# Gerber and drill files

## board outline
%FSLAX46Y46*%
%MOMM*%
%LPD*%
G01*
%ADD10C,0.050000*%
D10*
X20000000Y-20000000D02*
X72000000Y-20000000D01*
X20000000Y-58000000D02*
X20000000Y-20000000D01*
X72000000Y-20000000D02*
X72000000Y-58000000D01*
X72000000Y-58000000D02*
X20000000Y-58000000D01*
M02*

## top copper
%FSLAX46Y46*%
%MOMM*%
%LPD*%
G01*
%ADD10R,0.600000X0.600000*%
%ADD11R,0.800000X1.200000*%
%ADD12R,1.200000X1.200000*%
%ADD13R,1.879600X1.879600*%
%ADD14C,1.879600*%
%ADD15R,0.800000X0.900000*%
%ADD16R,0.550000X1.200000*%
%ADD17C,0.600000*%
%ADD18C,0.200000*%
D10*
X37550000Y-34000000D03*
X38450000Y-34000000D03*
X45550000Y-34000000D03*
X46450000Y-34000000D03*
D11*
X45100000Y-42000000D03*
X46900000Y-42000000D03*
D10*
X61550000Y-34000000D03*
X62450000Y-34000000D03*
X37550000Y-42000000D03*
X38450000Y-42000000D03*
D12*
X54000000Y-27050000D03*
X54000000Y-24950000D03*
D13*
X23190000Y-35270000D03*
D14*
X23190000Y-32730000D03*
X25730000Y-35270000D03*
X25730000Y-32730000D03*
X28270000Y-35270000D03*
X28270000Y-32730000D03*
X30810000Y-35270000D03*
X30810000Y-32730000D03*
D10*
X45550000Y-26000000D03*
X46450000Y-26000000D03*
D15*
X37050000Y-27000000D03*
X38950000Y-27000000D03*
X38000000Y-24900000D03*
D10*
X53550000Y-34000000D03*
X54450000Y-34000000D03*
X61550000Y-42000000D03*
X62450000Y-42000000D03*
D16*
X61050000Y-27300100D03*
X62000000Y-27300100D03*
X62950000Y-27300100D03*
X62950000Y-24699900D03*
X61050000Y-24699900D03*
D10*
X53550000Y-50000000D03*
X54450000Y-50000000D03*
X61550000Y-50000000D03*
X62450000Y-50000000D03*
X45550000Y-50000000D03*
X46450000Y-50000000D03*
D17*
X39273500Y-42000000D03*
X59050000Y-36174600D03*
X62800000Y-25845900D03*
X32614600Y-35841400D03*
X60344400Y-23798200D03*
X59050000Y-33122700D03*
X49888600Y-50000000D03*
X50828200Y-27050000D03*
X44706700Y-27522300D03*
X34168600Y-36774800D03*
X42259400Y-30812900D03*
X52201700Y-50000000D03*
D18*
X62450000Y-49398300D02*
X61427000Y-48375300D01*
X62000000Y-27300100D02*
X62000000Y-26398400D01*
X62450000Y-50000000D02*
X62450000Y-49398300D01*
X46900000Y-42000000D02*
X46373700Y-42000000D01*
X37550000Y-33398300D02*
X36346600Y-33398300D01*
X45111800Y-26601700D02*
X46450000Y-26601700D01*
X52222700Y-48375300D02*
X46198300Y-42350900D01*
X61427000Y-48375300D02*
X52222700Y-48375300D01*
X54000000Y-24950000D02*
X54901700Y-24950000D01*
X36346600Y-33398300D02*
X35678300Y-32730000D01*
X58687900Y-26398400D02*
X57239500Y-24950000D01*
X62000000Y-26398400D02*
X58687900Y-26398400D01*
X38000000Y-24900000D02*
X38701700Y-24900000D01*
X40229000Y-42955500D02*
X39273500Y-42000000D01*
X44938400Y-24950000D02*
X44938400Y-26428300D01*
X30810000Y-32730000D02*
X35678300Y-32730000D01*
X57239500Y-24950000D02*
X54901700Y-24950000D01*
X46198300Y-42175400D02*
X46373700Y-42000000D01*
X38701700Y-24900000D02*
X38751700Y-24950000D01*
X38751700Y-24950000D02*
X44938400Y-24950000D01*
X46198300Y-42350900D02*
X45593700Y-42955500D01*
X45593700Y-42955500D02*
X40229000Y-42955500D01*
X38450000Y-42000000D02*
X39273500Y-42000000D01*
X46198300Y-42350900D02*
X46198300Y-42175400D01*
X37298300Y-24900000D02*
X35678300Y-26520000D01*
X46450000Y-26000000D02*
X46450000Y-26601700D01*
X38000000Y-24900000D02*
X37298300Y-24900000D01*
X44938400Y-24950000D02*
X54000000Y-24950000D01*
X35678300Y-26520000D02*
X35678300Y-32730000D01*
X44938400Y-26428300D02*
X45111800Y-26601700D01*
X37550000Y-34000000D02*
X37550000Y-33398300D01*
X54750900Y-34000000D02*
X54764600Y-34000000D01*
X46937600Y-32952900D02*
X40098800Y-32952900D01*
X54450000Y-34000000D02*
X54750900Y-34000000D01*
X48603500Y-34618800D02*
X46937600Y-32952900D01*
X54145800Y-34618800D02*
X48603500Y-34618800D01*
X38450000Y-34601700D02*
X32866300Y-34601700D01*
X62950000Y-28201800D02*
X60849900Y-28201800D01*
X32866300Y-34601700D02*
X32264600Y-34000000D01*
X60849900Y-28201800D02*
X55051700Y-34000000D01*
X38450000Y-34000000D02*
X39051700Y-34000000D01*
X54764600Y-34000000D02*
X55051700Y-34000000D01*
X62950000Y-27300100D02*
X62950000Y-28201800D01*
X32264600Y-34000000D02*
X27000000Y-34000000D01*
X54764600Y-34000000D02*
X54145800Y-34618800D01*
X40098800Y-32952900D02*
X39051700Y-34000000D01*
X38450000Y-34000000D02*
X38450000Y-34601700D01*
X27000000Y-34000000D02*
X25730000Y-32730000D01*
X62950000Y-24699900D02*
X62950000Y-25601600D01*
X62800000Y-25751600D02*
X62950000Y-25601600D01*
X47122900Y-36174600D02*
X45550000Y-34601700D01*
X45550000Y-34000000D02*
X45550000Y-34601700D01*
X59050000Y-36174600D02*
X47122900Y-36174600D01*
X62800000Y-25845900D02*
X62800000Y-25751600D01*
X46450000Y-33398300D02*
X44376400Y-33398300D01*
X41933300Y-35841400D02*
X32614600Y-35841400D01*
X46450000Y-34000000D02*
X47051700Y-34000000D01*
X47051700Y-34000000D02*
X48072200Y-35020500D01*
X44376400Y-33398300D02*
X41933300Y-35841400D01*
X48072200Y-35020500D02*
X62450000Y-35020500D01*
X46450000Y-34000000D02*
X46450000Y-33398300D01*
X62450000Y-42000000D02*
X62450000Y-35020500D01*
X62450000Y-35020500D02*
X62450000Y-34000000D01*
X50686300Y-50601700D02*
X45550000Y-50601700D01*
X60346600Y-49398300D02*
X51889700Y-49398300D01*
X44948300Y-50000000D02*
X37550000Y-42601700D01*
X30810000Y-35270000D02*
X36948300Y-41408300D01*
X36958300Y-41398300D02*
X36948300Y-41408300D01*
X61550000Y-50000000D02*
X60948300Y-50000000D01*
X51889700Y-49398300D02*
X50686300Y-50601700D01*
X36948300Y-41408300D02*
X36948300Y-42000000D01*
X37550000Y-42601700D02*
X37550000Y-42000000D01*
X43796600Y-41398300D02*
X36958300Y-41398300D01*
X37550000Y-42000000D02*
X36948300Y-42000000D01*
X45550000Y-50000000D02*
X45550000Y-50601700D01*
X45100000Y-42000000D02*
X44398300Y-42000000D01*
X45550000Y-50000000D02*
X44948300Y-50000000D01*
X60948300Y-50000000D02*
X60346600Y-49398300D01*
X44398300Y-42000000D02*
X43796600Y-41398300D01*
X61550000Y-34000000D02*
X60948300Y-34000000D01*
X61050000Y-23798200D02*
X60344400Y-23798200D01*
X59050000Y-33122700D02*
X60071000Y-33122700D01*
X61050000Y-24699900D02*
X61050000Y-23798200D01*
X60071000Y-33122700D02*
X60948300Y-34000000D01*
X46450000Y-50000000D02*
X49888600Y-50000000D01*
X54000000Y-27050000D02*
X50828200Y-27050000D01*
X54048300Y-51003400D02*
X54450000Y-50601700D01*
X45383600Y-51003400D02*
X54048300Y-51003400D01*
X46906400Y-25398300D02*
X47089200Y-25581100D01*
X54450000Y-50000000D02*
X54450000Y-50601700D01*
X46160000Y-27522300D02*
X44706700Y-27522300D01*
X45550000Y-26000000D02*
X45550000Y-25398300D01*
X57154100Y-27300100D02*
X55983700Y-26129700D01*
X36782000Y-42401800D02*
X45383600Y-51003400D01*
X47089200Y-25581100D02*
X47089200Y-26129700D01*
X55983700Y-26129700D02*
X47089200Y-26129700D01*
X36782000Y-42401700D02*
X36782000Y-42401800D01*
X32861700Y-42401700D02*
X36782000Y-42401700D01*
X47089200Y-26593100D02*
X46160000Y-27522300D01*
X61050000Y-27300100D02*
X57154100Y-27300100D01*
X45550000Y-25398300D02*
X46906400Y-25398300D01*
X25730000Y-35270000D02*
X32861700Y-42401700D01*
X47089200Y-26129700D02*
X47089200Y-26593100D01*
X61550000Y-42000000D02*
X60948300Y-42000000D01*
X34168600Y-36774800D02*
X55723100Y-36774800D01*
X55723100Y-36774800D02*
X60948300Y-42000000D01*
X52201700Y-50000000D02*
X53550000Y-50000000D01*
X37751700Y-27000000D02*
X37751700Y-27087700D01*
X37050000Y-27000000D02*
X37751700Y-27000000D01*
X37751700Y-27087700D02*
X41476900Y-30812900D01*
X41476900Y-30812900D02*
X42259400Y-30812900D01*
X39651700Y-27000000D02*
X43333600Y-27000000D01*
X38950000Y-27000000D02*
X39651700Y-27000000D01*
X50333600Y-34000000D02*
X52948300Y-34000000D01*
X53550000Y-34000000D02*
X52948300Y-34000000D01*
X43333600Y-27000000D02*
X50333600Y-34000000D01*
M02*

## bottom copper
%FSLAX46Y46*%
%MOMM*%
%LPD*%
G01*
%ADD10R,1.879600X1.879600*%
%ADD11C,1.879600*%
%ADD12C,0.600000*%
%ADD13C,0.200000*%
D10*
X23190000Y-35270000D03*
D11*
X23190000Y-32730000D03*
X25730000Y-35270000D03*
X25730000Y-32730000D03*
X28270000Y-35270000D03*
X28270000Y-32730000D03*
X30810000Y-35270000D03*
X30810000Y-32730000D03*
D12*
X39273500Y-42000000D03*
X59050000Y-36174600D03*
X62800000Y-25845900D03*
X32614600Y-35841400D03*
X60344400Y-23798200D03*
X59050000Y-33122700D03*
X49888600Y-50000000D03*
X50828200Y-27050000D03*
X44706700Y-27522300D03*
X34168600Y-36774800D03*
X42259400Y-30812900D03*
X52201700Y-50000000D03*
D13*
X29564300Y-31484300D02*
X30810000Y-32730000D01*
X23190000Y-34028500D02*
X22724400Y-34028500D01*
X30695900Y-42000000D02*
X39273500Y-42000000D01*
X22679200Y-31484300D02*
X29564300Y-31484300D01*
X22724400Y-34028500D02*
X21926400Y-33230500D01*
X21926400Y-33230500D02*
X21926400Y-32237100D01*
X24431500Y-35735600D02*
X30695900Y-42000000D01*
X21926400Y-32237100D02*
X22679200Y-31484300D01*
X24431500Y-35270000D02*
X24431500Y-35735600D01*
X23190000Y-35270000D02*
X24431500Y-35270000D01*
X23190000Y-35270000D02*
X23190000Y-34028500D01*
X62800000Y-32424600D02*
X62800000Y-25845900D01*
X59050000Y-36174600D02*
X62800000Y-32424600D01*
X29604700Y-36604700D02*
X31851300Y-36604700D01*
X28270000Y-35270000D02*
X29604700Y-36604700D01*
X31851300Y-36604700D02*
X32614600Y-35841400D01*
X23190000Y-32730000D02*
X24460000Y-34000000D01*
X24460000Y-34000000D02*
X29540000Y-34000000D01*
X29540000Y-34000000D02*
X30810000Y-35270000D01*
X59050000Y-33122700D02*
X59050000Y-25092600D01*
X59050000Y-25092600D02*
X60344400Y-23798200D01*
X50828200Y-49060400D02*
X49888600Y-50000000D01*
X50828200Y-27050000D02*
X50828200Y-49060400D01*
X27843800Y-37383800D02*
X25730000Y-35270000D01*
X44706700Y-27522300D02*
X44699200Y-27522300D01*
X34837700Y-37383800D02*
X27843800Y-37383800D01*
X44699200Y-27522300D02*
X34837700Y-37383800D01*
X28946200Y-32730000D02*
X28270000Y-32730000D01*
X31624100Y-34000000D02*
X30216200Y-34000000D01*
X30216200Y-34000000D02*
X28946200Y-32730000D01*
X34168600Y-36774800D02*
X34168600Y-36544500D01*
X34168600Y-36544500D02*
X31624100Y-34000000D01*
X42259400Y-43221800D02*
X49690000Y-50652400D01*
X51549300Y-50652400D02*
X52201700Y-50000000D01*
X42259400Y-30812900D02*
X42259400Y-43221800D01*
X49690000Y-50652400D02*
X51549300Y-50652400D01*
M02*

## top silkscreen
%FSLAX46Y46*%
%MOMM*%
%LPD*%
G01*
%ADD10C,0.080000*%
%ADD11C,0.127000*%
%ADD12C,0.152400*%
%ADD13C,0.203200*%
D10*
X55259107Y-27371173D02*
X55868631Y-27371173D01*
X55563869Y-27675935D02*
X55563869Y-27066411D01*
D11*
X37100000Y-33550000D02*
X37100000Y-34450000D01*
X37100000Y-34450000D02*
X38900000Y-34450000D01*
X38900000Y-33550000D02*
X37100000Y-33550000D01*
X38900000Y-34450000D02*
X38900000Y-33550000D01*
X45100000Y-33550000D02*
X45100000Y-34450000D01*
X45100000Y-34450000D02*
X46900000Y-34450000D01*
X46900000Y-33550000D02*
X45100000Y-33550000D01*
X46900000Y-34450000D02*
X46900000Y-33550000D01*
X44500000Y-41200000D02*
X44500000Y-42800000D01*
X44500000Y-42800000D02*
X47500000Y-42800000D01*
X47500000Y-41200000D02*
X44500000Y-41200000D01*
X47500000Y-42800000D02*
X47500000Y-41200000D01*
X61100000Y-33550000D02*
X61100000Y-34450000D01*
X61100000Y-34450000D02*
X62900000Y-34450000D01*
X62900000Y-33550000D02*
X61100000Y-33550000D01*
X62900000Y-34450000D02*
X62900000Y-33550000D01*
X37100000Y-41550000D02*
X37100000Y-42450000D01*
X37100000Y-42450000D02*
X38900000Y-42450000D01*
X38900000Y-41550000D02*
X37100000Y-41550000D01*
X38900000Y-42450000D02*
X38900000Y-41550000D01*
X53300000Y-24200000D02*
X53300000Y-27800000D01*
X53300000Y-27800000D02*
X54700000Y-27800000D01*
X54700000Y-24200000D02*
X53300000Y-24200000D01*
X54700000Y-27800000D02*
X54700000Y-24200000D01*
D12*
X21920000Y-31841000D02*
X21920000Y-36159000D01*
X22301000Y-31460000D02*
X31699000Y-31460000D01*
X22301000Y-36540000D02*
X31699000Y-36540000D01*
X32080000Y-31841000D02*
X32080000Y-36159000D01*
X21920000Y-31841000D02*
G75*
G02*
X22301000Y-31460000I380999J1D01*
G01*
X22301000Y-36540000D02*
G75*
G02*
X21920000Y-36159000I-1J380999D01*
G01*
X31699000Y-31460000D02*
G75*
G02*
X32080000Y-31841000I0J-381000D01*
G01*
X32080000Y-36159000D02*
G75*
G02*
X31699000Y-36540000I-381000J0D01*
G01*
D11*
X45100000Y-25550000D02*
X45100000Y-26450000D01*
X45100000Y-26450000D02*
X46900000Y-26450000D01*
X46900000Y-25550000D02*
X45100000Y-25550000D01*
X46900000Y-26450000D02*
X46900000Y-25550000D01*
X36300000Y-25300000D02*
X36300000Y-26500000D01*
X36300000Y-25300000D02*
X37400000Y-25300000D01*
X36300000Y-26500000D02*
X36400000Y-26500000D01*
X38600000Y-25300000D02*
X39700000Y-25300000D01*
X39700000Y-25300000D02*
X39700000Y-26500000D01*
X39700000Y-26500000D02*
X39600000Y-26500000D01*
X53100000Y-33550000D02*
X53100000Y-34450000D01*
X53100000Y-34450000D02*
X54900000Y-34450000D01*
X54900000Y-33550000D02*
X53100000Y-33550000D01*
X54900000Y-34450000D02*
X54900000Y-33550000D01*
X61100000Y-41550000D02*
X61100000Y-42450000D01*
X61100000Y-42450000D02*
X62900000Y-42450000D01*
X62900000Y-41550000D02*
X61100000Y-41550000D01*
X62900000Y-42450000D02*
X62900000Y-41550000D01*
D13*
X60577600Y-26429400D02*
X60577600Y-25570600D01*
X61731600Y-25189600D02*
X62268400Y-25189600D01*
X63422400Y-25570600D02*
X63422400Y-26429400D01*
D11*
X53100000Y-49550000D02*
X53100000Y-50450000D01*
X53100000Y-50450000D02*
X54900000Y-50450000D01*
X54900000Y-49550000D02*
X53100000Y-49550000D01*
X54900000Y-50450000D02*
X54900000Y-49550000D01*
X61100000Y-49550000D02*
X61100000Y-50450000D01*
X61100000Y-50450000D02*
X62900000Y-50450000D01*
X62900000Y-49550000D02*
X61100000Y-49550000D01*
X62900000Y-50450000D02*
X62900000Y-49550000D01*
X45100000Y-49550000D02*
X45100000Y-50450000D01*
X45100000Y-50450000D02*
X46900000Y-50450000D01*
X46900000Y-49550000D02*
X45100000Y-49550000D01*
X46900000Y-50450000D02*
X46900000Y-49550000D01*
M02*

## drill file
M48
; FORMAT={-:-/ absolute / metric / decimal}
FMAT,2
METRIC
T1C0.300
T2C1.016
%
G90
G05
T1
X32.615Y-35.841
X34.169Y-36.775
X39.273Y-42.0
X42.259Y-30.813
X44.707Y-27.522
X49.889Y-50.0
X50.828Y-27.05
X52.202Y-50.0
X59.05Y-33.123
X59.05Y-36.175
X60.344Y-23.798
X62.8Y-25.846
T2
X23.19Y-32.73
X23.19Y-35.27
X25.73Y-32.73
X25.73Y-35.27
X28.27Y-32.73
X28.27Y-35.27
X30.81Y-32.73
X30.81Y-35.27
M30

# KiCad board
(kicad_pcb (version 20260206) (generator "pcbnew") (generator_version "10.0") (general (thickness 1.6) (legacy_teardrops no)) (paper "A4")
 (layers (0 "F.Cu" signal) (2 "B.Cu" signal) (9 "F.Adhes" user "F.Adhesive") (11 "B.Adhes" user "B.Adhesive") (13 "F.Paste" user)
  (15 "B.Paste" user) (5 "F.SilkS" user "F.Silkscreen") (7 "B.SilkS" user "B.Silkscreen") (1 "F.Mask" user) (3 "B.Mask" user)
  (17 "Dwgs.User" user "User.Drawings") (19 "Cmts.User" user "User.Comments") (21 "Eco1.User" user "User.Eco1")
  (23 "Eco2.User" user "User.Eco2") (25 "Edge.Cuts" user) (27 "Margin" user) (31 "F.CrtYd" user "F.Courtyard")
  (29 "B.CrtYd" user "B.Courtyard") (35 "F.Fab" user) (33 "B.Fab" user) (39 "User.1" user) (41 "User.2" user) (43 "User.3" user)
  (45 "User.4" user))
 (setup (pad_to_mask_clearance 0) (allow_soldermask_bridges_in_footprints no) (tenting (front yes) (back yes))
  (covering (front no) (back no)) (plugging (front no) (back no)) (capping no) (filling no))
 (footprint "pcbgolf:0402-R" (layer "F.Cu") (at 38 34)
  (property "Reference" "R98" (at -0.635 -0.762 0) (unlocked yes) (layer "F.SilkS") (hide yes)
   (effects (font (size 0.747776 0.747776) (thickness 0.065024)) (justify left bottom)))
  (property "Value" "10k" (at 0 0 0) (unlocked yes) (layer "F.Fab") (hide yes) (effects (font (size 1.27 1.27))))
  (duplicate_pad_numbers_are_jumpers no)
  (fp_line (start -0.9 -0.45) (end -0.9 0.45) (stroke (width 0.127) (type solid)) (layer "F.SilkS"))
  (fp_line (start -0.9 0.45) (end 0.9 0.45) (stroke (width 0.127) (type solid)) (layer "F.SilkS"))
  (fp_line (start 0.9 -0.45) (end -0.9 -0.45) (stroke (width 0.127) (type solid)) (layer "F.SilkS"))
  (fp_line (start 0.9 0.45) (end 0.9 -0.45) (stroke (width 0.127) (type solid)) (layer "F.SilkS"))
  (pad "1" smd rect (at -0.45 0) (size 0.6 0.6) (layers "F.Cu" "F.Mask" "F.Paste") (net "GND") (solder_mask_margin 0.0508)
   (solder_paste_margin 0) (thermal_bridge_angle 0))
  (pad "2" smd rect (at 0.45 0) (size 0.6 0.6) (layers "F.Cu" "F.Mask" "F.Paste") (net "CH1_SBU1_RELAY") (solder_mask_margin 0.0508)
   (solder_paste_margin 0) (thermal_bridge_angle 0)))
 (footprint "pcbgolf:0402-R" (layer "F.Cu") (at 46 34)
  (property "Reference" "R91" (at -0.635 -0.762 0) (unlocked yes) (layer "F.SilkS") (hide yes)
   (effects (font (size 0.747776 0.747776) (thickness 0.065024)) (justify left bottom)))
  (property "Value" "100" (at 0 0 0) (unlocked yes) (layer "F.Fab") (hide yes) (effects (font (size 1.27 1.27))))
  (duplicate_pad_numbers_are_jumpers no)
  (fp_line (start -0.9 -0.45) (end -0.9 0.45) (stroke (width 0.127) (type solid)) (layer "F.SilkS"))
  (fp_line (start -0.9 0.45) (end 0.9 0.45) (stroke (width 0.127) (type solid)) (layer "F.SilkS"))
  (fp_line (start 0.9 -0.45) (end -0.9 -0.45) (stroke (width 0.127) (type solid)) (layer "F.SilkS"))
  (fp_line (start 0.9 0.45) (end 0.9 -0.45) (stroke (width 0.127) (type solid)) (layer "F.SilkS"))
  (pad "1" smd rect (at -0.45 0) (size 0.6 0.6) (layers "F.Cu" "F.Mask" "F.Paste") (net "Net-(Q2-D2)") (solder_mask_margin 0.0508)
   (solder_paste_margin 0) (thermal_bridge_angle 0))
  (pad "2" smd rect (at 0.45 0) (size 0.6 0.6) (layers "F.Cu" "F.Mask" "F.Paste") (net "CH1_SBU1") (solder_mask_margin 0.0508)
   (solder_paste_margin 0) (thermal_bridge_angle 0)))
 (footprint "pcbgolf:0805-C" (layer "F.Cu") (at 46 42)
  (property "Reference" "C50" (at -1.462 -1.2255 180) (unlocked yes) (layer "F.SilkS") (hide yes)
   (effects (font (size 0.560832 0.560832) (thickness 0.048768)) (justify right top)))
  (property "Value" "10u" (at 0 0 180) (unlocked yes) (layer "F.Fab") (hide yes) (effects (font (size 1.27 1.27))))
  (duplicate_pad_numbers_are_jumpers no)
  (fp_line (start -1.5 -0.8) (end -1.5 0.8) (stroke (width 0.127) (type solid)) (layer "F.SilkS"))
  (fp_line (start -1.5 0.8) (end 1.5 0.8) (stroke (width 0.127) (type solid)) (layer "F.SilkS"))
  (fp_line (start 1.5 -0.8) (end -1.5 -0.8) (stroke (width 0.127) (type solid)) (layer "F.SilkS"))
  (fp_line (start 1.5 0.8) (end 1.5 -0.8) (stroke (width 0.127) (type solid)) (layer "F.SilkS"))
  (pad "1" smd rect (at -0.9 0) (size 0.8 1.2) (layers "F.Cu" "F.Mask" "F.Paste") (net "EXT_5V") (solder_mask_margin 0.0508)
   (solder_paste_margin 0) (thermal_bridge_angle 0))
  (pad "2" smd rect (at 0.9 0) (size 0.8 1.2) (layers "F.Cu" "F.Mask" "F.Paste") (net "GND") (solder_mask_margin 0.0508)
   (solder_paste_margin 0) (thermal_bridge_angle 0)))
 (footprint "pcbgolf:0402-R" (layer "F.Cu") (at 62 34)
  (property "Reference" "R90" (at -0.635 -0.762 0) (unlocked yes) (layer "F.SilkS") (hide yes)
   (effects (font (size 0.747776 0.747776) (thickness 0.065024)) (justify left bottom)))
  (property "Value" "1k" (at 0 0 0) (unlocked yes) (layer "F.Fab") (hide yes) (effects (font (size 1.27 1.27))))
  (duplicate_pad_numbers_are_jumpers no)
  (fp_line (start -0.9 -0.45) (end -0.9 0.45) (stroke (width 0.127) (type solid)) (layer "F.SilkS"))
  (fp_line (start -0.9 0.45) (end 0.9 0.45) (stroke (width 0.127) (type solid)) (layer "F.SilkS"))
  (fp_line (start 0.9 -0.45) (end -0.9 -0.45) (stroke (width 0.127) (type solid)) (layer "F.SilkS"))
  (fp_line (start 0.9 0.45) (end 0.9 -0.45) (stroke (width 0.127) (type solid)) (layer "F.SilkS"))
  (pad "1" smd rect (at -0.45 0) (size 0.6 0.6) (layers "F.Cu" "F.Mask" "F.Paste") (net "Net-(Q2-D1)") (solder_mask_margin 0.0508)
   (solder_paste_margin 0) (thermal_bridge_angle 0))
  (pad "2" smd rect (at 0.45 0) (size 0.6 0.6) (layers "F.Cu" "F.Mask" "F.Paste") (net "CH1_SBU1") (solder_mask_margin 0.0508)
   (solder_paste_margin 0) (thermal_bridge_angle 0)))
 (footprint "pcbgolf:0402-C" (layer "F.Cu") (at 38 42)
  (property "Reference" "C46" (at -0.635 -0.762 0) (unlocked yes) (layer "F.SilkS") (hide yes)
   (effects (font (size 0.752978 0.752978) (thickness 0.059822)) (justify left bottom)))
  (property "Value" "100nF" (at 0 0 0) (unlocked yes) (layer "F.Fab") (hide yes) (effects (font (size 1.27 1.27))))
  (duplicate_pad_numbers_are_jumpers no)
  (fp_line (start -0.9 -0.45) (end -0.9 0.45) (stroke (width 0.127) (type solid)) (layer "F.SilkS"))
  (fp_line (start -0.9 0.45) (end 0.9 0.45) (stroke (width 0.127) (type solid)) (layer "F.SilkS"))
  (fp_line (start 0.9 -0.45) (end -0.9 -0.45) (stroke (width 0.127) (type solid)) (layer "F.SilkS"))
  (fp_line (start 0.9 0.45) (end 0.9 -0.45) (stroke (width 0.127) (type solid)) (layer "F.SilkS"))
  (pad "1" smd rect (at -0.45 0) (size 0.6 0.6) (layers "F.Cu" "F.Mask" "F.Paste") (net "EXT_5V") (solder_mask_margin 0.0508)
   (solder_paste_margin 0) (thermal_bridge_angle 0))
  (pad "2" smd rect (at 0.45 0) (size 0.6 0.6) (layers "F.Cu" "F.Mask" "F.Paste") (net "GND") (solder_mask_margin 0.0508)
   (solder_paste_margin 0) (thermal_bridge_angle 0)))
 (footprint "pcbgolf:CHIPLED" (layer "F.Cu") (at 54 26)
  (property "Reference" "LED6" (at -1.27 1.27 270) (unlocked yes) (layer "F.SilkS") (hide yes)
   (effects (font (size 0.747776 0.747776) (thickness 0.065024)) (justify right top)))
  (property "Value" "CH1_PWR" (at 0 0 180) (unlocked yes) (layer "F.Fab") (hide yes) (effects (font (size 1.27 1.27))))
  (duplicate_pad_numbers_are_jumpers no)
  (fp_line (start -0.7 -1.8) (end -0.7 1.8) (stroke (width 0.127) (type solid)) (layer "F.SilkS"))
  (fp_line (start -0.7 1.8) (end 0.7 1.8) (stroke (width 0.127) (type solid)) (layer "F.SilkS"))
  (fp_line (start 0.7 -1.8) (end -0.7 -1.8) (stroke (width 0.127) (type solid)) (layer "F.SilkS"))
  (fp_line (start 0.7 1.8) (end 0.7 -1.8) (stroke (width 0.127) (type solid)) (layer "F.SilkS"))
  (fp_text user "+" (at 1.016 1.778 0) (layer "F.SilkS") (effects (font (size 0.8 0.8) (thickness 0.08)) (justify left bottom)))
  (pad "A" smd rect (at 0 1.05) (size 1.2 1.2) (layers "F.Cu" "F.Mask" "F.Paste") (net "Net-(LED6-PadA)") (solder_mask_margin 0.0508)
   (solder_paste_margin 0) (thermal_bridge_angle 0))
  (pad "C" smd rect (at 0 -1.05) (size 1.2 1.2) (layers "F.Cu" "F.Mask" "F.Paste") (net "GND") (solder_mask_margin 0.0508)
   (solder_paste_margin 0) (thermal_bridge_angle 0)))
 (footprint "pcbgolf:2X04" (layer "F.Cu") (at 27 34)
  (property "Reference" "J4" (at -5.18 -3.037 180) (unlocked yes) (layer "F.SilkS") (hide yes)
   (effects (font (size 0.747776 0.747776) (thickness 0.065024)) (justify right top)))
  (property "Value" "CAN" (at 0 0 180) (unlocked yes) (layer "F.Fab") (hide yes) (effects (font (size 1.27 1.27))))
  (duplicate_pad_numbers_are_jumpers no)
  (fp_line (start -5.08 -2.159) (end -5.08 2.159) (stroke (width 0.1524) (type solid)) (layer "F.SilkS"))
  (fp_line (start -4.699 -2.54) (end 4.699 -2.54) (stroke (width 0.1524) (type solid)) (layer "F.SilkS"))
  (fp_line (start -4.699 2.54) (end 4.699 2.54) (stroke (width 0.1524) (type solid)) (layer "F.SilkS"))
  (fp_line (start 5.08 -2.159) (end 5.08 2.159) (stroke (width 0.1524) (type solid)) (layer "F.SilkS"))
  (fp_arc (start -5.08 -2.159) (mid -4.968408 -2.428408) (end -4.699 -2.54) (stroke (width 0.1524) (type solid)) (layer "F.SilkS"))
  (fp_arc (start -4.699 2.54) (mid -4.968408 2.428408) (end -5.08 2.159) (stroke (width 0.1524) (type solid)) (layer "F.SilkS"))
  (fp_arc (start 4.699 -2.54) (mid 4.968408 -2.428408) (end 5.08 -2.159) (stroke (width 0.1524) (type solid)) (layer "F.SilkS"))
  (fp_arc (start 5.08 2.159) (mid 4.968408 2.428408) (end 4.699 2.54) (stroke (width 0.1524) (type solid)) (layer "F.SilkS"))
  (pad "1" thru_hole rect (at -3.81 1.27 90) (size 1.8796 1.8796) (drill 1.016) (layers "*.Cu" "*.Mask") (remove_unused_layers no)
   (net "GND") (solder_mask_margin 0.0508) (thermal_bridge_angle 0))
  (pad "2" thru_hole circle (at -3.81 -1.27 90) (size 1.8796 1.8796) (drill 1.016) (layers "*.Cu" "*.Mask") (remove_unused_layers no)
   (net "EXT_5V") (solder_mask_margin 0.0508) (thermal_bridge_angle 0))
  (pad "3" thru_hole circle (at -1.27 1.27 90) (size 1.8796 1.8796) (drill 1.016) (layers "*.Cu" "*.Mask") (remove_unused_layers no)
   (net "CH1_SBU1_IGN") (solder_mask_margin 0.0508) (thermal_bridge_angle 0))
  (pad "4" thru_hole circle (at -1.27 -1.27 90) (size 1.8796 1.8796) (drill 1.016) (layers "*.Cu" "*.Mask") (remove_unused_layers no)
   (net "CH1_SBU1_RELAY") (solder_mask_margin 0.0508) (thermal_bridge_angle 0))
  (pad "5" thru_hole circle (at 1.27 1.27 90) (size 1.8796 1.8796) (drill 1.016) (layers "*.Cu" "*.Mask") (remove_unused_layers no)
   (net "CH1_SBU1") (solder_mask_margin 0.0508) (thermal_bridge_angle 0))
  (pad "6" thru_hole circle (at 1.27 -1.27 90) (size 1.8796 1.8796) (drill 1.016) (layers "*.Cu" "*.Mask") (remove_unused_layers no)
   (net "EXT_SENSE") (solder_mask_margin 0.0508) (thermal_bridge_angle 0))
  (pad "7" thru_hole circle (at 3.81 1.27 90) (size 1.8796 1.8796) (drill 1.016) (layers "*.Cu" "*.Mask") (remove_unused_layers no)
   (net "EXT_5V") (solder_mask_margin 0.0508) (thermal_bridge_angle 0))
  (pad "8" thru_hole circle (at 3.81 -1.27 90) (size 1.8796 1.8796) (drill 1.016) (layers "*.Cu" "*.Mask") (remove_unused_layers no)
   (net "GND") (solder_mask_margin 0.0508) (thermal_bridge_angle 0)))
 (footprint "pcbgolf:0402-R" (layer "F.Cu") (at 46 26)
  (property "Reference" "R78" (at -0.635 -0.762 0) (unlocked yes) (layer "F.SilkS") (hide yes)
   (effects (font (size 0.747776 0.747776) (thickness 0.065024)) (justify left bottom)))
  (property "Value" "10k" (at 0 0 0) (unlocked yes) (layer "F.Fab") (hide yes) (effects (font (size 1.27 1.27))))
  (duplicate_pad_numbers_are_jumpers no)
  (fp_line (start -0.9 -0.45) (end -0.9 0.45) (stroke (width 0.127) (type solid)) (layer "F.SilkS"))
  (fp_line (start -0.9 0.45) (end 0.9 0.45) (stroke (width 0.127) (type solid)) (layer "F.SilkS"))
  (fp_line (start 0.9 -0.45) (end -0.9 -0.45) (stroke (width 0.127) (type solid)) (layer "F.SilkS"))
  (fp_line (start 0.9 0.45) (end 0.9 -0.45) (stroke (width 0.127) (type solid)) (layer "F.SilkS"))
  (pad "1" smd rect (at -0.45 0) (size 0.6 0.6) (layers "F.Cu" "F.Mask" "F.Paste") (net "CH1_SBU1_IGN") (solder_mask_margin 0.0508)
   (solder_paste_margin 0) (thermal_bridge_angle 0))
  (pad "2" smd rect (at 0.45 0) (size 0.6 0.6) (layers "F.Cu" "F.Mask" "F.Paste") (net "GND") (solder_mask_margin 0.0508)
   (solder_paste_margin 0) (thermal_bridge_angle 0)))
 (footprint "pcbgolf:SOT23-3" (layer "F.Cu") (at 38 26)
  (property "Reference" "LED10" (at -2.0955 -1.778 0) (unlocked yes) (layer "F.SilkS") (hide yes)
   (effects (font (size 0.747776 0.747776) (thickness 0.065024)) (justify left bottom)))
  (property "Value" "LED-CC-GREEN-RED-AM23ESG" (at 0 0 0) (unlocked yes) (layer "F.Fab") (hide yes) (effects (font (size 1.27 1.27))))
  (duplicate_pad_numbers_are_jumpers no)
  (fp_line (start -1.7 -0.7) (end -1.7 0.5) (stroke (width 0.127) (type solid)) (layer "F.SilkS"))
  (fp_line (start -1.7 -0.7) (end -0.6 -0.7) (stroke (width 0.127) (type solid)) (layer "F.SilkS"))
  (fp_line (start -1.7 0.5) (end -1.6 0.5) (stroke (width 0.127) (type solid)) (layer "F.SilkS"))
  (fp_line (start 0.6 -0.7) (end 1.7 -0.7) (stroke (width 0.127) (type solid)) (layer "F.SilkS"))
  (fp_line (start 1.7 -0.7) (end 1.7 0.5) (stroke (width 0.127) (type solid)) (layer "F.SilkS"))
  (fp_line (start 1.7 0.5) (end 1.6 0.5) (stroke (width 0.127) (type solid)) (layer "F.SilkS"))
  (pad "1" smd rect (at -0.95 1) (size 0.8 0.9) (layers "F.Cu" "F.Mask" "F.Paste") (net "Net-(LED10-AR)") (solder_mask_margin 0.0508)
   (solder_paste_margin 0) (thermal_bridge_angle 0))
  (pad "2" smd rect (at 0.95 1) (size 0.8 0.9) (layers "F.Cu" "F.Mask" "F.Paste") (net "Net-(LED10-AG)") (solder_mask_margin 0.0508)
   (solder_paste_margin 0) (thermal_bridge_angle 0))
  (pad "3" smd rect (at 0 -1.1) (size 0.8 0.9) (layers "F.Cu" "F.Mask" "F.Paste") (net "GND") (solder_mask_margin 0.0508)
   (solder_paste_margin 0) (thermal_bridge_angle 0)))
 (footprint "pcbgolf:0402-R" (layer "F.Cu") (at 54 34)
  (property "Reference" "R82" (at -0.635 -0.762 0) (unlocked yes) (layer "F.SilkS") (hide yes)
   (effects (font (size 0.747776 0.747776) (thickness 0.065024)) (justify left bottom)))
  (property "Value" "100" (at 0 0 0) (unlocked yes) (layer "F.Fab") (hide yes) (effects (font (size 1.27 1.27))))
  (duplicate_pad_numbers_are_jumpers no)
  (fp_line (start -0.9 -0.45) (end -0.9 0.45) (stroke (width 0.127) (type solid)) (layer "F.SilkS"))
  (fp_line (start -0.9 0.45) (end 0.9 0.45) (stroke (width 0.127) (type solid)) (layer "F.SilkS"))
  (fp_line (start 0.9 -0.45) (end -0.9 -0.45) (stroke (width 0.127) (type solid)) (layer "F.SilkS"))
  (fp_line (start 0.9 0.45) (end 0.9 -0.45) (stroke (width 0.127) (type solid)) (layer "F.SilkS"))
  (pad "1" smd rect (at -0.45 0) (size 0.6 0.6) (layers "F.Cu" "F.Mask" "F.Paste") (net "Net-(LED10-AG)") (solder_mask_margin 0.0508)
   (solder_paste_margin 0) (thermal_bridge_angle 0))
  (pad "2" smd rect (at 0.45 0) (size 0.6 0.6) (layers "F.Cu" "F.Mask" "F.Paste") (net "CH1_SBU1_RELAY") (solder_mask_margin 0.0508)
   (solder_paste_margin 0) (thermal_bridge_angle 0)))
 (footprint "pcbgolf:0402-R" (layer "F.Cu") (at 62 42)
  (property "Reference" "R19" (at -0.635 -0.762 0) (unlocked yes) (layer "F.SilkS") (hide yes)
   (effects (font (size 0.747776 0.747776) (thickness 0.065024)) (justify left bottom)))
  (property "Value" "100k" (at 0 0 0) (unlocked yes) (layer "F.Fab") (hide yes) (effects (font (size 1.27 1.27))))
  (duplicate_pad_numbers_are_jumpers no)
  (fp_line (start -0.9 -0.45) (end -0.9 0.45) (stroke (width 0.127) (type solid)) (layer "F.SilkS"))
  (fp_line (start -0.9 0.45) (end 0.9 0.45) (stroke (width 0.127) (type solid)) (layer "F.SilkS"))
  (fp_line (start 0.9 -0.45) (end -0.9 -0.45) (stroke (width 0.127) (type solid)) (layer "F.SilkS"))
  (fp_line (start 0.9 0.45) (end 0.9 -0.45) (stroke (width 0.127) (type solid)) (layer "F.SilkS"))
  (pad "1" smd rect (at -0.45 0) (size 0.6 0.6) (layers "F.Cu" "F.Mask" "F.Paste") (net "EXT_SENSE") (solder_mask_margin 0.0508)
   (solder_paste_margin 0) (thermal_bridge_angle 0))
  (pad "2" smd rect (at 0.45 0) (size 0.6 0.6) (layers "F.Cu" "F.Mask" "F.Paste") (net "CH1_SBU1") (solder_mask_margin 0.0508)
   (solder_paste_margin 0) (thermal_bridge_angle 0)))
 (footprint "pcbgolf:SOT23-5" (layer "F.Cu") (at 62 26)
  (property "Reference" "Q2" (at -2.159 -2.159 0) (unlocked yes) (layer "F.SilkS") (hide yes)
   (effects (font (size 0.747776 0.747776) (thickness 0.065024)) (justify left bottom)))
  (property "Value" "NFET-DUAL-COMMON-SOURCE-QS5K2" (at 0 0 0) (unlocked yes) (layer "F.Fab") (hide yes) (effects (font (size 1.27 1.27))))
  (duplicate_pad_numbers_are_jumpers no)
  (fp_line (start -1.4224 0.4294) (end -1.4224 -0.4294) (stroke (width 0.2032) (type solid)) (layer "F.SilkS"))
  (fp_line (start -0.2684 -0.8104) (end 0.2684 -0.8104) (stroke (width 0.2032) (type solid)) (layer "F.SilkS"))
  (fp_line (start 1.4224 -0.4294) (end 1.4224 0.4294) (stroke (width 0.2032) (type solid)) (layer "F.SilkS"))
  (pad "1" smd rect (at -0.95 1.3001) (size 0.55 1.2) (layers "F.Cu" "F.Mask" "F.Paste") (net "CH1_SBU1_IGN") (solder_mask_margin 0.0508)
   (solder_paste_margin 0) (thermal_bridge_angle 0))
  (pad "2" smd rect (at 0 1.3001) (size 0.55 1.2) (layers "F.Cu" "F.Mask" "F.Paste") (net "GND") (solder_mask_margin 0.0508)
   (solder_paste_margin 0) (thermal_bridge_angle 0))
  (pad "3" smd rect (at 0.95 1.3001) (size 0.55 1.2) (layers "F.Cu" "F.Mask" "F.Paste") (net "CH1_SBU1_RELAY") (solder_mask_margin 0.0508)
   (solder_paste_margin 0) (thermal_bridge_angle 0))
  (pad "4" smd rect (at 0.95 -1.3001) (size 0.55 1.2) (layers "F.Cu" "F.Mask" "F.Paste") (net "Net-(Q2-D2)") (solder_mask_margin 0.0508)
   (solder_paste_margin 0) (thermal_bridge_angle 0))
  (pad "5" smd rect (at -0.95 -1.3001) (size 0.55 1.2) (layers "F.Cu" "F.Mask" "F.Paste") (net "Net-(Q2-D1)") (solder_mask_margin 0.0508)
   (solder_paste_margin 0) (thermal_bridge_angle 0)))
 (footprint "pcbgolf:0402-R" (layer "F.Cu") (at 54 50)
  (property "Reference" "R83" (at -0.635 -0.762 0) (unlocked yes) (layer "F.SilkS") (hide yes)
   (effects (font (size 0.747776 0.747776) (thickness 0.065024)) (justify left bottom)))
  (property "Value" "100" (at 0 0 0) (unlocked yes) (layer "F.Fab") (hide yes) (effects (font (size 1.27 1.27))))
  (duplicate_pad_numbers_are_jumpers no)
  (fp_line (start -0.9 -0.45) (end -0.9 0.45) (stroke (width 0.127) (type solid)) (layer "F.SilkS"))
  (fp_line (start -0.9 0.45) (end 0.9 0.45) (stroke (width 0.127) (type solid)) (layer "F.SilkS"))
  (fp_line (start 0.9 -0.45) (end -0.9 -0.45) (stroke (width 0.127) (type solid)) (layer "F.SilkS"))
  (fp_line (start 0.9 0.45) (end 0.9 -0.45) (stroke (width 0.127) (type solid)) (layer "F.SilkS"))
  (pad "1" smd rect (at -0.45 0) (size 0.6 0.6) (layers "F.Cu" "F.Mask" "F.Paste") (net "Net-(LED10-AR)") (solder_mask_margin 0.0508)
   (solder_paste_margin 0) (thermal_bridge_angle 0))
  (pad "2" smd rect (at 0.45 0) (size 0.6 0.6) (layers "F.Cu" "F.Mask" "F.Paste") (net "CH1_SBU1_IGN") (solder_mask_margin 0.0508)
   (solder_paste_margin 0) (thermal_bridge_angle 0)))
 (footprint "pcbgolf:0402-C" (layer "F.Cu") (at 62 50)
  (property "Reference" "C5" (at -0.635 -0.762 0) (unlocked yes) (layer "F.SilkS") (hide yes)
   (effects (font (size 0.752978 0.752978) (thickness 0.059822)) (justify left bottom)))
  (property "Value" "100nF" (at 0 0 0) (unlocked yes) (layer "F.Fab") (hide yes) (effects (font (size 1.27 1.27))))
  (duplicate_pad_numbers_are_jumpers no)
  (fp_line (start -0.9 -0.45) (end -0.9 0.45) (stroke (width 0.127) (type solid)) (layer "F.SilkS"))
  (fp_line (start -0.9 0.45) (end 0.9 0.45) (stroke (width 0.127) (type solid)) (layer "F.SilkS"))
  (fp_line (start 0.9 -0.45) (end -0.9 -0.45) (stroke (width 0.127) (type solid)) (layer "F.SilkS"))
  (fp_line (start 0.9 0.45) (end 0.9 -0.45) (stroke (width 0.127) (type solid)) (layer "F.SilkS"))
  (pad "1" smd rect (at -0.45 0) (size 0.6 0.6) (layers "F.Cu" "F.Mask" "F.Paste") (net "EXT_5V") (solder_mask_margin 0.0508)
   (solder_paste_margin 0) (thermal_bridge_angle 0))
  (pad "2" smd rect (at 0.45 0) (size 0.6 0.6) (layers "F.Cu" "F.Mask" "F.Paste") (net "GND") (solder_mask_margin 0.0508)
   (solder_paste_margin 0) (thermal_bridge_angle 0)))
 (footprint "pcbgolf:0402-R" (layer "F.Cu") (at 46 50)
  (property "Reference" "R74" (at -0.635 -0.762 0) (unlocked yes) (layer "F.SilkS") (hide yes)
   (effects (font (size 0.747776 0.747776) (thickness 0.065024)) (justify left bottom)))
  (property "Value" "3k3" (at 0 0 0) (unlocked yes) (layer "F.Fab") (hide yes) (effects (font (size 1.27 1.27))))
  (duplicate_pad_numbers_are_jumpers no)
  (fp_line (start -0.9 -0.45) (end -0.9 0.45) (stroke (width 0.127) (type solid)) (layer "F.SilkS"))
  (fp_line (start -0.9 0.45) (end 0.9 0.45) (stroke (width 0.127) (type solid)) (layer "F.SilkS"))
  (fp_line (start 0.9 -0.45) (end -0.9 -0.45) (stroke (width 0.127) (type solid)) (layer "F.SilkS"))
  (fp_line (start 0.9 0.45) (end 0.9 -0.45) (stroke (width 0.127) (type solid)) (layer "F.SilkS"))
  (pad "1" smd rect (at -0.45 0) (size 0.6 0.6) (layers "F.Cu" "F.Mask" "F.Paste") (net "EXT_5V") (solder_mask_margin 0.0508)
   (solder_paste_margin 0) (thermal_bridge_angle 0))
  (pad "2" smd rect (at 0.45 0) (size 0.6 0.6) (layers "F.Cu" "F.Mask" "F.Paste") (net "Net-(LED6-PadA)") (solder_mask_margin 0.0508)
   (solder_paste_margin 0) (thermal_bridge_angle 0)))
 (gr_line (start 20 20) (end 72 20) (stroke (width 0.05) (type default)) (layer "Edge.Cuts"))
 (gr_line (start 20 58) (end 20 20) (stroke (width 0.05) (type default)) (layer "Edge.Cuts"))
 (gr_line (start 72 20) (end 72 58) (stroke (width 0.05) (type default)) (layer "Edge.Cuts"))
 (gr_line (start 72 58) (end 20 58) (stroke (width 0.05) (type default)) (layer "Edge.Cuts"))
 (segment (start 62.45 49.3983) (end 61.427 48.3753) (width 0.2) (layer "F.Cu") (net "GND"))
 (segment (start 62 27.3001) (end 62 26.3984) (width 0.2) (layer "F.Cu") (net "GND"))
 (segment (start 62.45 50) (end 62.45 49.3983) (width 0.2) (layer "F.Cu") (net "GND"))
 (segment (start 46.9 42) (end 46.3737 42) (width 0.2) (layer "F.Cu") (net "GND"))
 (segment (start 37.55 33.3983) (end 36.3466 33.3983) (width 0.2) (layer "F.Cu") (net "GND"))
 (segment (start 45.1118 26.6017) (end 46.45 26.6017) (width 0.2) (layer "F.Cu") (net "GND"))
 (segment (start 52.2227 48.3753) (end 46.1983 42.3509) (width 0.2) (layer "F.Cu") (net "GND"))
 (segment (start 61.427 48.3753) (end 52.2227 48.3753) (width 0.2) (layer "F.Cu") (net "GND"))
 (segment (start 54 24.95) (end 54.9017 24.95) (width 0.2) (layer "F.Cu") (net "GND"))
 (segment (start 36.3466 33.3983) (end 35.6783 32.73) (width 0.2) (layer "F.Cu") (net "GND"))
 (segment (start 58.6879 26.3984) (end 57.2395 24.95) (width 0.2) (layer "F.Cu") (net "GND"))
 (segment (start 62 26.3984) (end 58.6879 26.3984) (width 0.2) (layer "F.Cu") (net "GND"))
 (segment (start 38 24.9) (end 38.7017 24.9) (width 0.2) (layer "F.Cu") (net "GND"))
 (segment (start 40.229 42.9555) (end 39.2735 42) (width 0.2) (layer "F.Cu") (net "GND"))
 (segment (start 44.9384 24.95) (end 44.9384 26.4283) (width 0.2) (layer "F.Cu") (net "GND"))
 (segment (start 30.81 32.73) (end 35.6783 32.73) (width 0.2) (layer "F.Cu") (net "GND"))
 (segment (start 57.2395 24.95) (end 54.9017 24.95) (width 0.2) (layer "F.Cu") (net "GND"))
 (segment (start 46.1983 42.1754) (end 46.3737 42) (width 0.2) (layer "F.Cu") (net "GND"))
 (segment (start 38.7017 24.9) (end 38.7517 24.95) (width 0.2) (layer "F.Cu") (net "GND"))
 (segment (start 38.7517 24.95) (end 44.9384 24.95) (width 0.2) (layer "F.Cu") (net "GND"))
 (segment (start 46.1983 42.3509) (end 45.5937 42.9555) (width 0.2) (layer "F.Cu") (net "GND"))
 (segment (start 45.5937 42.9555) (end 40.229 42.9555) (width 0.2) (layer "F.Cu") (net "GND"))
 (segment (start 38.45 42) (end 39.2735 42) (width 0.2) (layer "F.Cu") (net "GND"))
 (segment (start 46.1983 42.3509) (end 46.1983 42.1754) (width 0.2) (layer "F.Cu") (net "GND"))
 (segment (start 37.2983 24.9) (end 35.6783 26.52) (width 0.2) (layer "F.Cu") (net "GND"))
 (segment (start 46.45 26) (end 46.45 26.6017) (width 0.2) (layer "F.Cu") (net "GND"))
 (segment (start 38 24.9) (end 37.2983 24.9) (width 0.2) (layer "F.Cu") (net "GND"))
 (segment (start 44.9384 24.95) (end 54 24.95) (width 0.2) (layer "F.Cu") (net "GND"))
 (segment (start 35.6783 26.52) (end 35.6783 32.73) (width 0.2) (layer "F.Cu") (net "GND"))
 (segment (start 44.9384 26.4283) (end 45.1118 26.6017) (width 0.2) (layer "F.Cu") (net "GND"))
 (segment (start 37.55 34) (end 37.55 33.3983) (width 0.2) (layer "F.Cu") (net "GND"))
 (via (at 39.2735 42) (size 0.6) (drill 0.3) (layers "F.Cu" "B.Cu") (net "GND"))
 (segment (start 29.5643 31.4843) (end 30.81 32.73) (width 0.2) (layer "B.Cu") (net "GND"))
 (segment (start 23.19 34.0285) (end 22.7244 34.0285) (width 0.2) (layer "B.Cu") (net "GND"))
 (segment (start 30.6959 42) (end 39.2735 42) (width 0.2) (layer "B.Cu") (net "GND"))
 (segment (start 22.6792 31.4843) (end 29.5643 31.4843) (width 0.2) (layer "B.Cu") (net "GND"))
 (segment (start 22.7244 34.0285) (end 21.9264 33.2305) (width 0.2) (layer "B.Cu") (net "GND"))
 (segment (start 21.9264 33.2305) (end 21.9264 32.2371) (width 0.2) (layer "B.Cu") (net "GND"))
 (segment (start 24.4315 35.7356) (end 30.6959 42) (width 0.2) (layer "B.Cu") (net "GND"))
 (segment (start 21.9264 32.2371) (end 22.6792 31.4843) (width 0.2) (layer "B.Cu") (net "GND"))
 (segment (start 24.4315 35.27) (end 24.4315 35.7356) (width 0.2) (layer "B.Cu") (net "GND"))
 (segment (start 23.19 35.27) (end 24.4315 35.27) (width 0.2) (layer "B.Cu") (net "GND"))
 (segment (start 23.19 35.27) (end 23.19 34.0285) (width 0.2) (layer "B.Cu") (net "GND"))
 (segment (start 54.7509 34) (end 54.7646 34) (width 0.2) (layer "F.Cu") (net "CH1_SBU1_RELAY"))
 (segment (start 46.9376 32.9529) (end 40.0988 32.9529) (width 0.2) (layer "F.Cu") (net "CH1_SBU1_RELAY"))
 (segment (start 54.45 34) (end 54.7509 34) (width 0.2) (layer "F.Cu") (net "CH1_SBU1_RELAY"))
 (segment (start 48.6035 34.6188) (end 46.9376 32.9529) (width 0.2) (layer "F.Cu") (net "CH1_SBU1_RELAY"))
 (segment (start 54.1458 34.6188) (end 48.6035 34.6188) (width 0.2) (layer "F.Cu") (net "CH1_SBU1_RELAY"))
 (segment (start 38.45 34.6017) (end 32.8663 34.6017) (width 0.2) (layer "F.Cu") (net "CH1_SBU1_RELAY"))
 (segment (start 62.95 28.2018) (end 60.8499 28.2018) (width 0.2) (layer "F.Cu") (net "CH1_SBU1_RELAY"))
 (segment (start 32.8663 34.6017) (end 32.2646 34) (width 0.2) (layer "F.Cu") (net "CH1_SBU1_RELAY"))
 (segment (start 60.8499 28.2018) (end 55.0517 34) (width 0.2) (layer "F.Cu") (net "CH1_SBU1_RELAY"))
 (segment (start 38.45 34) (end 39.0517 34) (width 0.2) (layer "F.Cu") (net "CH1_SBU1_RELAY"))
 (segment (start 54.7646 34) (end 55.0517 34) (width 0.2) (layer "F.Cu") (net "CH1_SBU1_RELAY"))
 (segment (start 62.95 27.3001) (end 62.95 28.2018) (width 0.2) (layer "F.Cu") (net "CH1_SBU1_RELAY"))
 (segment (start 32.2646 34) (end 27 34) (width 0.2) (layer "F.Cu") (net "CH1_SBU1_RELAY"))
 (segment (start 54.7646 34) (end 54.1458 34.6188) (width 0.2) (layer "F.Cu") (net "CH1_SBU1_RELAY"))
 (segment (start 40.0988 32.9529) (end 39.0517 34) (width 0.2) (layer "F.Cu") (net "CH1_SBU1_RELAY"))
 (segment (start 38.45 34) (end 38.45 34.6017) (width 0.2) (layer "F.Cu") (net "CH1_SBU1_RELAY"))
 (segment (start 27 34) (end 25.73 32.73) (width 0.2) (layer "F.Cu") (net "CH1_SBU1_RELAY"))
 (segment (start 62.95 24.6999) (end 62.95 25.6016) (width 0.2) (layer "F.Cu") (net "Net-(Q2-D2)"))
 (segment (start 62.8 25.7516) (end 62.95 25.6016) (width 0.2) (layer "F.Cu") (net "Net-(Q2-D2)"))
 (segment (start 47.1229 36.1746) (end 45.55 34.6017) (width 0.2) (layer "F.Cu") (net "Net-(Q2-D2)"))
 (segment (start 45.55 34) (end 45.55 34.6017) (width 0.2) (layer "F.Cu") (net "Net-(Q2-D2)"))
 (segment (start 59.05 36.1746) (end 47.1229 36.1746) (width 0.2) (layer "F.Cu") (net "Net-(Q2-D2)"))
 (segment (start 62.8 25.8459) (end 62.8 25.7516) (width 0.2) (layer "F.Cu") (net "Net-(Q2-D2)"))
 (via (at 59.05 36.1746) (size 0.6) (drill 0.3) (layers "F.Cu" "B.Cu") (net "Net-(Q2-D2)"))
 (via (at 62.8 25.8459) (size 0.6) (drill 0.3) (layers "F.Cu" "B.Cu") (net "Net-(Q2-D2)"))
 (segment (start 62.8 32.4246) (end 62.8 25.8459) (width 0.2) (layer "B.Cu") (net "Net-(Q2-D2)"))
 (segment (start 59.05 36.1746) (end 62.8 32.4246) (width 0.2) (layer "B.Cu") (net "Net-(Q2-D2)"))
 (segment (start 46.45 33.3983) (end 44.3764 33.3983) (width 0.2) (layer "F.Cu") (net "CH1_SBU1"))
 (segment (start 41.9333 35.8414) (end 32.6146 35.8414) (width 0.2) (layer "F.Cu") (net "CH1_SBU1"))
 (segment (start 46.45 34) (end 47.0517 34) (width 0.2) (layer "F.Cu") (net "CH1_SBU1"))
 (segment (start 47.0517 34) (end 48.0722 35.0205) (width 0.2) (layer "F.Cu") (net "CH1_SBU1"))
 (segment (start 44.3764 33.3983) (end 41.9333 35.8414) (width 0.2) (layer "F.Cu") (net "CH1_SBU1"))
 (segment (start 48.0722 35.0205) (end 62.45 35.0205) (width 0.2) (layer "F.Cu") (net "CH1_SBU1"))
 (segment (start 46.45 34) (end 46.45 33.3983) (width 0.2) (layer "F.Cu") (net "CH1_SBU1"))
 (segment (start 62.45 42) (end 62.45 35.0205) (width 0.2) (layer "F.Cu") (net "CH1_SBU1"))
 (segment (start 62.45 35.0205) (end 62.45 34) (width 0.2) (layer "F.Cu") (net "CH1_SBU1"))
 (via (at 32.6146 35.8414) (size 0.6) (drill 0.3) (layers "F.Cu" "B.Cu") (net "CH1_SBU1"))
 (segment (start 29.6047 36.6047) (end 31.8513 36.6047) (width 0.2) (layer "B.Cu") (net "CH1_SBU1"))
 (segment (start 28.27 35.27) (end 29.6047 36.6047) (width 0.2) (layer "B.Cu") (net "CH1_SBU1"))
 (segment (start 31.8513 36.6047) (end 32.6146 35.8414) (width 0.2) (layer "B.Cu") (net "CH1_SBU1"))
 (segment (start 50.6863 50.6017) (end 45.55 50.6017) (width 0.2) (layer "F.Cu") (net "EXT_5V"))
 (segment (start 60.3466 49.3983) (end 51.8897 49.3983) (width 0.2) (layer "F.Cu") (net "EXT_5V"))
 (segment (start 44.9483 50) (end 37.55 42.6017) (width 0.2) (layer "F.Cu") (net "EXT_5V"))
 (segment (start 30.81 35.27) (end 36.9483 41.4083) (width 0.2) (layer "F.Cu") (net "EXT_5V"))
 (segment (start 36.9583 41.3983) (end 36.9483 41.4083) (width 0.2) (layer "F.Cu") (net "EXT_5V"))
 (segment (start 61.55 50) (end 60.9483 50) (width 0.2) (layer "F.Cu") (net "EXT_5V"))
 (segment (start 51.8897 49.3983) (end 50.6863 50.6017) (width 0.2) (layer "F.Cu") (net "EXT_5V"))
 (segment (start 36.9483 41.4083) (end 36.9483 42) (width 0.2) (layer "F.Cu") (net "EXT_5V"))
 (segment (start 37.55 42.6017) (end 37.55 42) (width 0.2) (layer "F.Cu") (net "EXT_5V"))
 (segment (start 43.7966 41.3983) (end 36.9583 41.3983) (width 0.2) (layer "F.Cu") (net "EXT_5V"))
 (segment (start 37.55 42) (end 36.9483 42) (width 0.2) (layer "F.Cu") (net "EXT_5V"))
 (segment (start 45.55 50) (end 45.55 50.6017) (width 0.2) (layer "F.Cu") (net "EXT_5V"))
 (segment (start 45.1 42) (end 44.3983 42) (width 0.2) (layer "F.Cu") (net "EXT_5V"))
 (segment (start 45.55 50) (end 44.9483 50) (width 0.2) (layer "F.Cu") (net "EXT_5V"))
 (segment (start 60.9483 50) (end 60.3466 49.3983) (width 0.2) (layer "F.Cu") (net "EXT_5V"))
 (segment (start 44.3983 42) (end 43.7966 41.3983) (width 0.2) (layer "F.Cu") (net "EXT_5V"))
 (segment (start 23.19 32.73) (end 24.46 34) (width 0.2) (layer "B.Cu") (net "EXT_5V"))
 (segment (start 24.46 34) (end 29.54 34) (width 0.2) (layer "B.Cu") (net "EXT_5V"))
 (segment (start 29.54 34) (end 30.81 35.27) (width 0.2) (layer "B.Cu") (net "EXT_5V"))
 (segment (start 61.55 34) (end 60.9483 34) (width 0.2) (layer "F.Cu") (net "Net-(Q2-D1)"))
 (segment (start 61.05 23.7982) (end 60.3444 23.7982) (width 0.2) (layer "F.Cu") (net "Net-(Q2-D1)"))
 (segment (start 59.05 33.1227) (end 60.071 33.1227) (width 0.2) (layer "F.Cu") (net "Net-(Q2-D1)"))
 (segment (start 61.05 24.6999) (end 61.05 23.7982) (width 0.2) (layer "F.Cu") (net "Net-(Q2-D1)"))
 (segment (start 60.071 33.1227) (end 60.9483 34) (width 0.2) (layer "F.Cu") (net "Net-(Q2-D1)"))
 (via (at 60.3444 23.7982) (size 0.6) (drill 0.3) (layers "F.Cu" "B.Cu") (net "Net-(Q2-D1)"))
 (via (at 59.05 33.1227) (size 0.6) (drill 0.3) (layers "F.Cu" "B.Cu") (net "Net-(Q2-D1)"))
 (segment (start 59.05 33.1227) (end 59.05 25.0926) (width 0.2) (layer "B.Cu") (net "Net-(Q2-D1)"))
 (segment (start 59.05 25.0926) (end 60.3444 23.7982) (width 0.2) (layer "B.Cu") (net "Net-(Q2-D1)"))
 (segment (start 46.45 50) (end 49.8886 50) (width 0.2) (layer "F.Cu") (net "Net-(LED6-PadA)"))
 (segment (start 54 27.05) (end 50.8282 27.05) (width 0.2) (layer "F.Cu") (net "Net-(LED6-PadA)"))
 (via (at 49.8886 50) (size 0.6) (drill 0.3) (layers "F.Cu" "B.Cu") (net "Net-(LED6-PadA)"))
 (via (at 50.8282 27.05) (size 0.6) (drill 0.3) (layers "F.Cu" "B.Cu") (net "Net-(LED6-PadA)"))
 (segment (start 50.8282 49.0604) (end 49.8886 50) (width 0.2) (layer "B.Cu") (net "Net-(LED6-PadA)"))
 (segment (start 50.8282 27.05) (end 50.8282 49.0604) (width 0.2) (layer "B.Cu") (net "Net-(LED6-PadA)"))
 (segment (start 54.0483 51.0034) (end 54.45 50.6017) (width 0.2) (layer "F.Cu") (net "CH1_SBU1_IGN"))
 (segment (start 45.3836 51.0034) (end 54.0483 51.0034) (width 0.2) (layer "F.Cu") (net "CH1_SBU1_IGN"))
 (segment (start 46.9064 25.3983) (end 47.0892 25.5811) (width 0.2) (layer "F.Cu") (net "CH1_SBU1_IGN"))
 (segment (start 54.45 50) (end 54.45 50.6017) (width 0.2) (layer "F.Cu") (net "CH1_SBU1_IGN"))
 (segment (start 46.16 27.5223) (end 44.7067 27.5223) (width 0.2) (layer "F.Cu") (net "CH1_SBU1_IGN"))
 (segment (start 45.55 26) (end 45.55 25.3983) (width 0.2) (layer "F.Cu") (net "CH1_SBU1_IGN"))
 (segment (start 57.1541 27.3001) (end 55.9837 26.1297) (width 0.2) (layer "F.Cu") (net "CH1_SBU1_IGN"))
 (segment (start 36.782 42.4018) (end 45.3836 51.0034) (width 0.2) (layer "F.Cu") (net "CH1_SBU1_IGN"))
 (segment (start 47.0892 25.5811) (end 47.0892 26.1297) (width 0.2) (layer "F.Cu") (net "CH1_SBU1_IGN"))
 (segment (start 55.9837 26.1297) (end 47.0892 26.1297) (width 0.2) (layer "F.Cu") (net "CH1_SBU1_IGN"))
 (segment (start 36.782 42.4017) (end 36.782 42.4018) (width 0.2) (layer "F.Cu") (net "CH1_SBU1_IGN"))
 (segment (start 32.8617 42.4017) (end 36.782 42.4017) (width 0.2) (layer "F.Cu") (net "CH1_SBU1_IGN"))
 (segment (start 47.0892 26.5931) (end 46.16 27.5223) (width 0.2) (layer "F.Cu") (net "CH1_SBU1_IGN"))
 (segment (start 61.05 27.3001) (end 57.1541 27.3001) (width 0.2) (layer "F.Cu") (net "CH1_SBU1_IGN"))
 (segment (start 45.55 25.3983) (end 46.9064 25.3983) (width 0.2) (layer "F.Cu") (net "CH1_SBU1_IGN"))
 (segment (start 25.73 35.27) (end 32.8617 42.4017) (width 0.2) (layer "F.Cu") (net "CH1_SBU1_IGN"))
 (segment (start 47.0892 26.1297) (end 47.0892 26.5931) (width 0.2) (layer "F.Cu") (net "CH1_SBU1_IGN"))
 (via (at 44.7067 27.5223) (size 0.6) (drill 0.3) (layers "F.Cu" "B.Cu") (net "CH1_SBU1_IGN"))
 (segment (start 27.8438 37.3838) (end 25.73 35.27) (width 0.2) (layer "B.Cu") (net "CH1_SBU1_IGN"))
 (segment (start 44.7067 27.5223) (end 44.6992 27.5223) (width 0.2) (layer "B.Cu") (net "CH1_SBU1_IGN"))
 (segment (start 34.8377 37.3838) (end 27.8438 37.3838) (width 0.2) (layer "B.Cu") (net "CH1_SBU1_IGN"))
 (segment (start 44.6992 27.5223) (end 34.8377 37.3838) (width 0.2) (layer "B.Cu") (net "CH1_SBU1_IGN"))
 (segment (start 61.55 42) (end 60.9483 42) (width 0.2) (layer "F.Cu") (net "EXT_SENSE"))
 (segment (start 34.1686 36.7748) (end 55.7231 36.7748) (width 0.2) (layer "F.Cu") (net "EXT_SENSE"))
 (segment (start 55.7231 36.7748) (end 60.9483 42) (width 0.2) (layer "F.Cu") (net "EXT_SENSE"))
 (via (at 34.1686 36.7748) (size 0.6) (drill 0.3) (layers "F.Cu" "B.Cu") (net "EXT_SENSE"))
 (segment (start 28.9462 32.73) (end 28.27 32.73) (width 0.2) (layer "B.Cu") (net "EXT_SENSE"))
 (segment (start 31.6241 34) (end 30.2162 34) (width 0.2) (layer "B.Cu") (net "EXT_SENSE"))
 (segment (start 30.2162 34) (end 28.9462 32.73) (width 0.2) (layer "B.Cu") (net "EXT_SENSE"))
 (segment (start 34.1686 36.7748) (end 34.1686 36.5445) (width 0.2) (layer "B.Cu") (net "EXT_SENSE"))
 (segment (start 34.1686 36.5445) (end 31.6241 34) (width 0.2) (layer "B.Cu") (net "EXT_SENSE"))
 (segment (start 52.2017 50) (end 53.55 50) (width 0.2) (layer "F.Cu") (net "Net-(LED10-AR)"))
 (segment (start 37.7517 27) (end 37.7517 27.0877) (width 0.2) (layer "F.Cu") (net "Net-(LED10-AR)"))
 (segment (start 37.05 27) (end 37.7517 27) (width 0.2) (layer "F.Cu") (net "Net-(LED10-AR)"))
 (segment (start 37.7517 27.0877) (end 41.4769 30.8129) (width 0.2) (layer "F.Cu") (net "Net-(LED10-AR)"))
 (segment (start 41.4769 30.8129) (end 42.2594 30.8129) (width 0.2) (layer "F.Cu") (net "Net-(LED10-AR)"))
 (via (at 42.2594 30.8129) (size 0.6) (drill 0.3) (layers "F.Cu" "B.Cu") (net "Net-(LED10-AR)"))
 (via (at 52.2017 50) (size 0.6) (drill 0.3) (layers "F.Cu" "B.Cu") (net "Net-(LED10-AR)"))
 (segment (start 42.2594 43.2218) (end 49.69 50.6524) (width 0.2) (layer "B.Cu") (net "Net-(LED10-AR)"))
 (segment (start 51.5493 50.6524) (end 52.2017 50) (width 0.2) (layer "B.Cu") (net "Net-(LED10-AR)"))
 (segment (start 42.2594 30.8129) (end 42.2594 43.2218) (width 0.2) (layer "B.Cu") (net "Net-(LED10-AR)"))
 (segment (start 49.69 50.6524) (end 51.5493 50.6524) (width 0.2) (layer "B.Cu") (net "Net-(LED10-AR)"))
 (segment (start 39.6517 27) (end 43.3336 27) (width 0.2) (layer "F.Cu") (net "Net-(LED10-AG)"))
 (segment (start 38.95 27) (end 39.6517 27) (width 0.2) (layer "F.Cu") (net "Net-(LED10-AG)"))
 (segment (start 50.3336 34) (end 52.9483 34) (width 0.2) (layer "F.Cu") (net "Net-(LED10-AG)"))
 (segment (start 53.55 34) (end 52.9483 34) (width 0.2) (layer "F.Cu") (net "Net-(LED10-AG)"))
 (segment (start 43.3336 27) (end 50.3336 34) (width 0.2) (layer "F.Cu") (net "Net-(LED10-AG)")))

